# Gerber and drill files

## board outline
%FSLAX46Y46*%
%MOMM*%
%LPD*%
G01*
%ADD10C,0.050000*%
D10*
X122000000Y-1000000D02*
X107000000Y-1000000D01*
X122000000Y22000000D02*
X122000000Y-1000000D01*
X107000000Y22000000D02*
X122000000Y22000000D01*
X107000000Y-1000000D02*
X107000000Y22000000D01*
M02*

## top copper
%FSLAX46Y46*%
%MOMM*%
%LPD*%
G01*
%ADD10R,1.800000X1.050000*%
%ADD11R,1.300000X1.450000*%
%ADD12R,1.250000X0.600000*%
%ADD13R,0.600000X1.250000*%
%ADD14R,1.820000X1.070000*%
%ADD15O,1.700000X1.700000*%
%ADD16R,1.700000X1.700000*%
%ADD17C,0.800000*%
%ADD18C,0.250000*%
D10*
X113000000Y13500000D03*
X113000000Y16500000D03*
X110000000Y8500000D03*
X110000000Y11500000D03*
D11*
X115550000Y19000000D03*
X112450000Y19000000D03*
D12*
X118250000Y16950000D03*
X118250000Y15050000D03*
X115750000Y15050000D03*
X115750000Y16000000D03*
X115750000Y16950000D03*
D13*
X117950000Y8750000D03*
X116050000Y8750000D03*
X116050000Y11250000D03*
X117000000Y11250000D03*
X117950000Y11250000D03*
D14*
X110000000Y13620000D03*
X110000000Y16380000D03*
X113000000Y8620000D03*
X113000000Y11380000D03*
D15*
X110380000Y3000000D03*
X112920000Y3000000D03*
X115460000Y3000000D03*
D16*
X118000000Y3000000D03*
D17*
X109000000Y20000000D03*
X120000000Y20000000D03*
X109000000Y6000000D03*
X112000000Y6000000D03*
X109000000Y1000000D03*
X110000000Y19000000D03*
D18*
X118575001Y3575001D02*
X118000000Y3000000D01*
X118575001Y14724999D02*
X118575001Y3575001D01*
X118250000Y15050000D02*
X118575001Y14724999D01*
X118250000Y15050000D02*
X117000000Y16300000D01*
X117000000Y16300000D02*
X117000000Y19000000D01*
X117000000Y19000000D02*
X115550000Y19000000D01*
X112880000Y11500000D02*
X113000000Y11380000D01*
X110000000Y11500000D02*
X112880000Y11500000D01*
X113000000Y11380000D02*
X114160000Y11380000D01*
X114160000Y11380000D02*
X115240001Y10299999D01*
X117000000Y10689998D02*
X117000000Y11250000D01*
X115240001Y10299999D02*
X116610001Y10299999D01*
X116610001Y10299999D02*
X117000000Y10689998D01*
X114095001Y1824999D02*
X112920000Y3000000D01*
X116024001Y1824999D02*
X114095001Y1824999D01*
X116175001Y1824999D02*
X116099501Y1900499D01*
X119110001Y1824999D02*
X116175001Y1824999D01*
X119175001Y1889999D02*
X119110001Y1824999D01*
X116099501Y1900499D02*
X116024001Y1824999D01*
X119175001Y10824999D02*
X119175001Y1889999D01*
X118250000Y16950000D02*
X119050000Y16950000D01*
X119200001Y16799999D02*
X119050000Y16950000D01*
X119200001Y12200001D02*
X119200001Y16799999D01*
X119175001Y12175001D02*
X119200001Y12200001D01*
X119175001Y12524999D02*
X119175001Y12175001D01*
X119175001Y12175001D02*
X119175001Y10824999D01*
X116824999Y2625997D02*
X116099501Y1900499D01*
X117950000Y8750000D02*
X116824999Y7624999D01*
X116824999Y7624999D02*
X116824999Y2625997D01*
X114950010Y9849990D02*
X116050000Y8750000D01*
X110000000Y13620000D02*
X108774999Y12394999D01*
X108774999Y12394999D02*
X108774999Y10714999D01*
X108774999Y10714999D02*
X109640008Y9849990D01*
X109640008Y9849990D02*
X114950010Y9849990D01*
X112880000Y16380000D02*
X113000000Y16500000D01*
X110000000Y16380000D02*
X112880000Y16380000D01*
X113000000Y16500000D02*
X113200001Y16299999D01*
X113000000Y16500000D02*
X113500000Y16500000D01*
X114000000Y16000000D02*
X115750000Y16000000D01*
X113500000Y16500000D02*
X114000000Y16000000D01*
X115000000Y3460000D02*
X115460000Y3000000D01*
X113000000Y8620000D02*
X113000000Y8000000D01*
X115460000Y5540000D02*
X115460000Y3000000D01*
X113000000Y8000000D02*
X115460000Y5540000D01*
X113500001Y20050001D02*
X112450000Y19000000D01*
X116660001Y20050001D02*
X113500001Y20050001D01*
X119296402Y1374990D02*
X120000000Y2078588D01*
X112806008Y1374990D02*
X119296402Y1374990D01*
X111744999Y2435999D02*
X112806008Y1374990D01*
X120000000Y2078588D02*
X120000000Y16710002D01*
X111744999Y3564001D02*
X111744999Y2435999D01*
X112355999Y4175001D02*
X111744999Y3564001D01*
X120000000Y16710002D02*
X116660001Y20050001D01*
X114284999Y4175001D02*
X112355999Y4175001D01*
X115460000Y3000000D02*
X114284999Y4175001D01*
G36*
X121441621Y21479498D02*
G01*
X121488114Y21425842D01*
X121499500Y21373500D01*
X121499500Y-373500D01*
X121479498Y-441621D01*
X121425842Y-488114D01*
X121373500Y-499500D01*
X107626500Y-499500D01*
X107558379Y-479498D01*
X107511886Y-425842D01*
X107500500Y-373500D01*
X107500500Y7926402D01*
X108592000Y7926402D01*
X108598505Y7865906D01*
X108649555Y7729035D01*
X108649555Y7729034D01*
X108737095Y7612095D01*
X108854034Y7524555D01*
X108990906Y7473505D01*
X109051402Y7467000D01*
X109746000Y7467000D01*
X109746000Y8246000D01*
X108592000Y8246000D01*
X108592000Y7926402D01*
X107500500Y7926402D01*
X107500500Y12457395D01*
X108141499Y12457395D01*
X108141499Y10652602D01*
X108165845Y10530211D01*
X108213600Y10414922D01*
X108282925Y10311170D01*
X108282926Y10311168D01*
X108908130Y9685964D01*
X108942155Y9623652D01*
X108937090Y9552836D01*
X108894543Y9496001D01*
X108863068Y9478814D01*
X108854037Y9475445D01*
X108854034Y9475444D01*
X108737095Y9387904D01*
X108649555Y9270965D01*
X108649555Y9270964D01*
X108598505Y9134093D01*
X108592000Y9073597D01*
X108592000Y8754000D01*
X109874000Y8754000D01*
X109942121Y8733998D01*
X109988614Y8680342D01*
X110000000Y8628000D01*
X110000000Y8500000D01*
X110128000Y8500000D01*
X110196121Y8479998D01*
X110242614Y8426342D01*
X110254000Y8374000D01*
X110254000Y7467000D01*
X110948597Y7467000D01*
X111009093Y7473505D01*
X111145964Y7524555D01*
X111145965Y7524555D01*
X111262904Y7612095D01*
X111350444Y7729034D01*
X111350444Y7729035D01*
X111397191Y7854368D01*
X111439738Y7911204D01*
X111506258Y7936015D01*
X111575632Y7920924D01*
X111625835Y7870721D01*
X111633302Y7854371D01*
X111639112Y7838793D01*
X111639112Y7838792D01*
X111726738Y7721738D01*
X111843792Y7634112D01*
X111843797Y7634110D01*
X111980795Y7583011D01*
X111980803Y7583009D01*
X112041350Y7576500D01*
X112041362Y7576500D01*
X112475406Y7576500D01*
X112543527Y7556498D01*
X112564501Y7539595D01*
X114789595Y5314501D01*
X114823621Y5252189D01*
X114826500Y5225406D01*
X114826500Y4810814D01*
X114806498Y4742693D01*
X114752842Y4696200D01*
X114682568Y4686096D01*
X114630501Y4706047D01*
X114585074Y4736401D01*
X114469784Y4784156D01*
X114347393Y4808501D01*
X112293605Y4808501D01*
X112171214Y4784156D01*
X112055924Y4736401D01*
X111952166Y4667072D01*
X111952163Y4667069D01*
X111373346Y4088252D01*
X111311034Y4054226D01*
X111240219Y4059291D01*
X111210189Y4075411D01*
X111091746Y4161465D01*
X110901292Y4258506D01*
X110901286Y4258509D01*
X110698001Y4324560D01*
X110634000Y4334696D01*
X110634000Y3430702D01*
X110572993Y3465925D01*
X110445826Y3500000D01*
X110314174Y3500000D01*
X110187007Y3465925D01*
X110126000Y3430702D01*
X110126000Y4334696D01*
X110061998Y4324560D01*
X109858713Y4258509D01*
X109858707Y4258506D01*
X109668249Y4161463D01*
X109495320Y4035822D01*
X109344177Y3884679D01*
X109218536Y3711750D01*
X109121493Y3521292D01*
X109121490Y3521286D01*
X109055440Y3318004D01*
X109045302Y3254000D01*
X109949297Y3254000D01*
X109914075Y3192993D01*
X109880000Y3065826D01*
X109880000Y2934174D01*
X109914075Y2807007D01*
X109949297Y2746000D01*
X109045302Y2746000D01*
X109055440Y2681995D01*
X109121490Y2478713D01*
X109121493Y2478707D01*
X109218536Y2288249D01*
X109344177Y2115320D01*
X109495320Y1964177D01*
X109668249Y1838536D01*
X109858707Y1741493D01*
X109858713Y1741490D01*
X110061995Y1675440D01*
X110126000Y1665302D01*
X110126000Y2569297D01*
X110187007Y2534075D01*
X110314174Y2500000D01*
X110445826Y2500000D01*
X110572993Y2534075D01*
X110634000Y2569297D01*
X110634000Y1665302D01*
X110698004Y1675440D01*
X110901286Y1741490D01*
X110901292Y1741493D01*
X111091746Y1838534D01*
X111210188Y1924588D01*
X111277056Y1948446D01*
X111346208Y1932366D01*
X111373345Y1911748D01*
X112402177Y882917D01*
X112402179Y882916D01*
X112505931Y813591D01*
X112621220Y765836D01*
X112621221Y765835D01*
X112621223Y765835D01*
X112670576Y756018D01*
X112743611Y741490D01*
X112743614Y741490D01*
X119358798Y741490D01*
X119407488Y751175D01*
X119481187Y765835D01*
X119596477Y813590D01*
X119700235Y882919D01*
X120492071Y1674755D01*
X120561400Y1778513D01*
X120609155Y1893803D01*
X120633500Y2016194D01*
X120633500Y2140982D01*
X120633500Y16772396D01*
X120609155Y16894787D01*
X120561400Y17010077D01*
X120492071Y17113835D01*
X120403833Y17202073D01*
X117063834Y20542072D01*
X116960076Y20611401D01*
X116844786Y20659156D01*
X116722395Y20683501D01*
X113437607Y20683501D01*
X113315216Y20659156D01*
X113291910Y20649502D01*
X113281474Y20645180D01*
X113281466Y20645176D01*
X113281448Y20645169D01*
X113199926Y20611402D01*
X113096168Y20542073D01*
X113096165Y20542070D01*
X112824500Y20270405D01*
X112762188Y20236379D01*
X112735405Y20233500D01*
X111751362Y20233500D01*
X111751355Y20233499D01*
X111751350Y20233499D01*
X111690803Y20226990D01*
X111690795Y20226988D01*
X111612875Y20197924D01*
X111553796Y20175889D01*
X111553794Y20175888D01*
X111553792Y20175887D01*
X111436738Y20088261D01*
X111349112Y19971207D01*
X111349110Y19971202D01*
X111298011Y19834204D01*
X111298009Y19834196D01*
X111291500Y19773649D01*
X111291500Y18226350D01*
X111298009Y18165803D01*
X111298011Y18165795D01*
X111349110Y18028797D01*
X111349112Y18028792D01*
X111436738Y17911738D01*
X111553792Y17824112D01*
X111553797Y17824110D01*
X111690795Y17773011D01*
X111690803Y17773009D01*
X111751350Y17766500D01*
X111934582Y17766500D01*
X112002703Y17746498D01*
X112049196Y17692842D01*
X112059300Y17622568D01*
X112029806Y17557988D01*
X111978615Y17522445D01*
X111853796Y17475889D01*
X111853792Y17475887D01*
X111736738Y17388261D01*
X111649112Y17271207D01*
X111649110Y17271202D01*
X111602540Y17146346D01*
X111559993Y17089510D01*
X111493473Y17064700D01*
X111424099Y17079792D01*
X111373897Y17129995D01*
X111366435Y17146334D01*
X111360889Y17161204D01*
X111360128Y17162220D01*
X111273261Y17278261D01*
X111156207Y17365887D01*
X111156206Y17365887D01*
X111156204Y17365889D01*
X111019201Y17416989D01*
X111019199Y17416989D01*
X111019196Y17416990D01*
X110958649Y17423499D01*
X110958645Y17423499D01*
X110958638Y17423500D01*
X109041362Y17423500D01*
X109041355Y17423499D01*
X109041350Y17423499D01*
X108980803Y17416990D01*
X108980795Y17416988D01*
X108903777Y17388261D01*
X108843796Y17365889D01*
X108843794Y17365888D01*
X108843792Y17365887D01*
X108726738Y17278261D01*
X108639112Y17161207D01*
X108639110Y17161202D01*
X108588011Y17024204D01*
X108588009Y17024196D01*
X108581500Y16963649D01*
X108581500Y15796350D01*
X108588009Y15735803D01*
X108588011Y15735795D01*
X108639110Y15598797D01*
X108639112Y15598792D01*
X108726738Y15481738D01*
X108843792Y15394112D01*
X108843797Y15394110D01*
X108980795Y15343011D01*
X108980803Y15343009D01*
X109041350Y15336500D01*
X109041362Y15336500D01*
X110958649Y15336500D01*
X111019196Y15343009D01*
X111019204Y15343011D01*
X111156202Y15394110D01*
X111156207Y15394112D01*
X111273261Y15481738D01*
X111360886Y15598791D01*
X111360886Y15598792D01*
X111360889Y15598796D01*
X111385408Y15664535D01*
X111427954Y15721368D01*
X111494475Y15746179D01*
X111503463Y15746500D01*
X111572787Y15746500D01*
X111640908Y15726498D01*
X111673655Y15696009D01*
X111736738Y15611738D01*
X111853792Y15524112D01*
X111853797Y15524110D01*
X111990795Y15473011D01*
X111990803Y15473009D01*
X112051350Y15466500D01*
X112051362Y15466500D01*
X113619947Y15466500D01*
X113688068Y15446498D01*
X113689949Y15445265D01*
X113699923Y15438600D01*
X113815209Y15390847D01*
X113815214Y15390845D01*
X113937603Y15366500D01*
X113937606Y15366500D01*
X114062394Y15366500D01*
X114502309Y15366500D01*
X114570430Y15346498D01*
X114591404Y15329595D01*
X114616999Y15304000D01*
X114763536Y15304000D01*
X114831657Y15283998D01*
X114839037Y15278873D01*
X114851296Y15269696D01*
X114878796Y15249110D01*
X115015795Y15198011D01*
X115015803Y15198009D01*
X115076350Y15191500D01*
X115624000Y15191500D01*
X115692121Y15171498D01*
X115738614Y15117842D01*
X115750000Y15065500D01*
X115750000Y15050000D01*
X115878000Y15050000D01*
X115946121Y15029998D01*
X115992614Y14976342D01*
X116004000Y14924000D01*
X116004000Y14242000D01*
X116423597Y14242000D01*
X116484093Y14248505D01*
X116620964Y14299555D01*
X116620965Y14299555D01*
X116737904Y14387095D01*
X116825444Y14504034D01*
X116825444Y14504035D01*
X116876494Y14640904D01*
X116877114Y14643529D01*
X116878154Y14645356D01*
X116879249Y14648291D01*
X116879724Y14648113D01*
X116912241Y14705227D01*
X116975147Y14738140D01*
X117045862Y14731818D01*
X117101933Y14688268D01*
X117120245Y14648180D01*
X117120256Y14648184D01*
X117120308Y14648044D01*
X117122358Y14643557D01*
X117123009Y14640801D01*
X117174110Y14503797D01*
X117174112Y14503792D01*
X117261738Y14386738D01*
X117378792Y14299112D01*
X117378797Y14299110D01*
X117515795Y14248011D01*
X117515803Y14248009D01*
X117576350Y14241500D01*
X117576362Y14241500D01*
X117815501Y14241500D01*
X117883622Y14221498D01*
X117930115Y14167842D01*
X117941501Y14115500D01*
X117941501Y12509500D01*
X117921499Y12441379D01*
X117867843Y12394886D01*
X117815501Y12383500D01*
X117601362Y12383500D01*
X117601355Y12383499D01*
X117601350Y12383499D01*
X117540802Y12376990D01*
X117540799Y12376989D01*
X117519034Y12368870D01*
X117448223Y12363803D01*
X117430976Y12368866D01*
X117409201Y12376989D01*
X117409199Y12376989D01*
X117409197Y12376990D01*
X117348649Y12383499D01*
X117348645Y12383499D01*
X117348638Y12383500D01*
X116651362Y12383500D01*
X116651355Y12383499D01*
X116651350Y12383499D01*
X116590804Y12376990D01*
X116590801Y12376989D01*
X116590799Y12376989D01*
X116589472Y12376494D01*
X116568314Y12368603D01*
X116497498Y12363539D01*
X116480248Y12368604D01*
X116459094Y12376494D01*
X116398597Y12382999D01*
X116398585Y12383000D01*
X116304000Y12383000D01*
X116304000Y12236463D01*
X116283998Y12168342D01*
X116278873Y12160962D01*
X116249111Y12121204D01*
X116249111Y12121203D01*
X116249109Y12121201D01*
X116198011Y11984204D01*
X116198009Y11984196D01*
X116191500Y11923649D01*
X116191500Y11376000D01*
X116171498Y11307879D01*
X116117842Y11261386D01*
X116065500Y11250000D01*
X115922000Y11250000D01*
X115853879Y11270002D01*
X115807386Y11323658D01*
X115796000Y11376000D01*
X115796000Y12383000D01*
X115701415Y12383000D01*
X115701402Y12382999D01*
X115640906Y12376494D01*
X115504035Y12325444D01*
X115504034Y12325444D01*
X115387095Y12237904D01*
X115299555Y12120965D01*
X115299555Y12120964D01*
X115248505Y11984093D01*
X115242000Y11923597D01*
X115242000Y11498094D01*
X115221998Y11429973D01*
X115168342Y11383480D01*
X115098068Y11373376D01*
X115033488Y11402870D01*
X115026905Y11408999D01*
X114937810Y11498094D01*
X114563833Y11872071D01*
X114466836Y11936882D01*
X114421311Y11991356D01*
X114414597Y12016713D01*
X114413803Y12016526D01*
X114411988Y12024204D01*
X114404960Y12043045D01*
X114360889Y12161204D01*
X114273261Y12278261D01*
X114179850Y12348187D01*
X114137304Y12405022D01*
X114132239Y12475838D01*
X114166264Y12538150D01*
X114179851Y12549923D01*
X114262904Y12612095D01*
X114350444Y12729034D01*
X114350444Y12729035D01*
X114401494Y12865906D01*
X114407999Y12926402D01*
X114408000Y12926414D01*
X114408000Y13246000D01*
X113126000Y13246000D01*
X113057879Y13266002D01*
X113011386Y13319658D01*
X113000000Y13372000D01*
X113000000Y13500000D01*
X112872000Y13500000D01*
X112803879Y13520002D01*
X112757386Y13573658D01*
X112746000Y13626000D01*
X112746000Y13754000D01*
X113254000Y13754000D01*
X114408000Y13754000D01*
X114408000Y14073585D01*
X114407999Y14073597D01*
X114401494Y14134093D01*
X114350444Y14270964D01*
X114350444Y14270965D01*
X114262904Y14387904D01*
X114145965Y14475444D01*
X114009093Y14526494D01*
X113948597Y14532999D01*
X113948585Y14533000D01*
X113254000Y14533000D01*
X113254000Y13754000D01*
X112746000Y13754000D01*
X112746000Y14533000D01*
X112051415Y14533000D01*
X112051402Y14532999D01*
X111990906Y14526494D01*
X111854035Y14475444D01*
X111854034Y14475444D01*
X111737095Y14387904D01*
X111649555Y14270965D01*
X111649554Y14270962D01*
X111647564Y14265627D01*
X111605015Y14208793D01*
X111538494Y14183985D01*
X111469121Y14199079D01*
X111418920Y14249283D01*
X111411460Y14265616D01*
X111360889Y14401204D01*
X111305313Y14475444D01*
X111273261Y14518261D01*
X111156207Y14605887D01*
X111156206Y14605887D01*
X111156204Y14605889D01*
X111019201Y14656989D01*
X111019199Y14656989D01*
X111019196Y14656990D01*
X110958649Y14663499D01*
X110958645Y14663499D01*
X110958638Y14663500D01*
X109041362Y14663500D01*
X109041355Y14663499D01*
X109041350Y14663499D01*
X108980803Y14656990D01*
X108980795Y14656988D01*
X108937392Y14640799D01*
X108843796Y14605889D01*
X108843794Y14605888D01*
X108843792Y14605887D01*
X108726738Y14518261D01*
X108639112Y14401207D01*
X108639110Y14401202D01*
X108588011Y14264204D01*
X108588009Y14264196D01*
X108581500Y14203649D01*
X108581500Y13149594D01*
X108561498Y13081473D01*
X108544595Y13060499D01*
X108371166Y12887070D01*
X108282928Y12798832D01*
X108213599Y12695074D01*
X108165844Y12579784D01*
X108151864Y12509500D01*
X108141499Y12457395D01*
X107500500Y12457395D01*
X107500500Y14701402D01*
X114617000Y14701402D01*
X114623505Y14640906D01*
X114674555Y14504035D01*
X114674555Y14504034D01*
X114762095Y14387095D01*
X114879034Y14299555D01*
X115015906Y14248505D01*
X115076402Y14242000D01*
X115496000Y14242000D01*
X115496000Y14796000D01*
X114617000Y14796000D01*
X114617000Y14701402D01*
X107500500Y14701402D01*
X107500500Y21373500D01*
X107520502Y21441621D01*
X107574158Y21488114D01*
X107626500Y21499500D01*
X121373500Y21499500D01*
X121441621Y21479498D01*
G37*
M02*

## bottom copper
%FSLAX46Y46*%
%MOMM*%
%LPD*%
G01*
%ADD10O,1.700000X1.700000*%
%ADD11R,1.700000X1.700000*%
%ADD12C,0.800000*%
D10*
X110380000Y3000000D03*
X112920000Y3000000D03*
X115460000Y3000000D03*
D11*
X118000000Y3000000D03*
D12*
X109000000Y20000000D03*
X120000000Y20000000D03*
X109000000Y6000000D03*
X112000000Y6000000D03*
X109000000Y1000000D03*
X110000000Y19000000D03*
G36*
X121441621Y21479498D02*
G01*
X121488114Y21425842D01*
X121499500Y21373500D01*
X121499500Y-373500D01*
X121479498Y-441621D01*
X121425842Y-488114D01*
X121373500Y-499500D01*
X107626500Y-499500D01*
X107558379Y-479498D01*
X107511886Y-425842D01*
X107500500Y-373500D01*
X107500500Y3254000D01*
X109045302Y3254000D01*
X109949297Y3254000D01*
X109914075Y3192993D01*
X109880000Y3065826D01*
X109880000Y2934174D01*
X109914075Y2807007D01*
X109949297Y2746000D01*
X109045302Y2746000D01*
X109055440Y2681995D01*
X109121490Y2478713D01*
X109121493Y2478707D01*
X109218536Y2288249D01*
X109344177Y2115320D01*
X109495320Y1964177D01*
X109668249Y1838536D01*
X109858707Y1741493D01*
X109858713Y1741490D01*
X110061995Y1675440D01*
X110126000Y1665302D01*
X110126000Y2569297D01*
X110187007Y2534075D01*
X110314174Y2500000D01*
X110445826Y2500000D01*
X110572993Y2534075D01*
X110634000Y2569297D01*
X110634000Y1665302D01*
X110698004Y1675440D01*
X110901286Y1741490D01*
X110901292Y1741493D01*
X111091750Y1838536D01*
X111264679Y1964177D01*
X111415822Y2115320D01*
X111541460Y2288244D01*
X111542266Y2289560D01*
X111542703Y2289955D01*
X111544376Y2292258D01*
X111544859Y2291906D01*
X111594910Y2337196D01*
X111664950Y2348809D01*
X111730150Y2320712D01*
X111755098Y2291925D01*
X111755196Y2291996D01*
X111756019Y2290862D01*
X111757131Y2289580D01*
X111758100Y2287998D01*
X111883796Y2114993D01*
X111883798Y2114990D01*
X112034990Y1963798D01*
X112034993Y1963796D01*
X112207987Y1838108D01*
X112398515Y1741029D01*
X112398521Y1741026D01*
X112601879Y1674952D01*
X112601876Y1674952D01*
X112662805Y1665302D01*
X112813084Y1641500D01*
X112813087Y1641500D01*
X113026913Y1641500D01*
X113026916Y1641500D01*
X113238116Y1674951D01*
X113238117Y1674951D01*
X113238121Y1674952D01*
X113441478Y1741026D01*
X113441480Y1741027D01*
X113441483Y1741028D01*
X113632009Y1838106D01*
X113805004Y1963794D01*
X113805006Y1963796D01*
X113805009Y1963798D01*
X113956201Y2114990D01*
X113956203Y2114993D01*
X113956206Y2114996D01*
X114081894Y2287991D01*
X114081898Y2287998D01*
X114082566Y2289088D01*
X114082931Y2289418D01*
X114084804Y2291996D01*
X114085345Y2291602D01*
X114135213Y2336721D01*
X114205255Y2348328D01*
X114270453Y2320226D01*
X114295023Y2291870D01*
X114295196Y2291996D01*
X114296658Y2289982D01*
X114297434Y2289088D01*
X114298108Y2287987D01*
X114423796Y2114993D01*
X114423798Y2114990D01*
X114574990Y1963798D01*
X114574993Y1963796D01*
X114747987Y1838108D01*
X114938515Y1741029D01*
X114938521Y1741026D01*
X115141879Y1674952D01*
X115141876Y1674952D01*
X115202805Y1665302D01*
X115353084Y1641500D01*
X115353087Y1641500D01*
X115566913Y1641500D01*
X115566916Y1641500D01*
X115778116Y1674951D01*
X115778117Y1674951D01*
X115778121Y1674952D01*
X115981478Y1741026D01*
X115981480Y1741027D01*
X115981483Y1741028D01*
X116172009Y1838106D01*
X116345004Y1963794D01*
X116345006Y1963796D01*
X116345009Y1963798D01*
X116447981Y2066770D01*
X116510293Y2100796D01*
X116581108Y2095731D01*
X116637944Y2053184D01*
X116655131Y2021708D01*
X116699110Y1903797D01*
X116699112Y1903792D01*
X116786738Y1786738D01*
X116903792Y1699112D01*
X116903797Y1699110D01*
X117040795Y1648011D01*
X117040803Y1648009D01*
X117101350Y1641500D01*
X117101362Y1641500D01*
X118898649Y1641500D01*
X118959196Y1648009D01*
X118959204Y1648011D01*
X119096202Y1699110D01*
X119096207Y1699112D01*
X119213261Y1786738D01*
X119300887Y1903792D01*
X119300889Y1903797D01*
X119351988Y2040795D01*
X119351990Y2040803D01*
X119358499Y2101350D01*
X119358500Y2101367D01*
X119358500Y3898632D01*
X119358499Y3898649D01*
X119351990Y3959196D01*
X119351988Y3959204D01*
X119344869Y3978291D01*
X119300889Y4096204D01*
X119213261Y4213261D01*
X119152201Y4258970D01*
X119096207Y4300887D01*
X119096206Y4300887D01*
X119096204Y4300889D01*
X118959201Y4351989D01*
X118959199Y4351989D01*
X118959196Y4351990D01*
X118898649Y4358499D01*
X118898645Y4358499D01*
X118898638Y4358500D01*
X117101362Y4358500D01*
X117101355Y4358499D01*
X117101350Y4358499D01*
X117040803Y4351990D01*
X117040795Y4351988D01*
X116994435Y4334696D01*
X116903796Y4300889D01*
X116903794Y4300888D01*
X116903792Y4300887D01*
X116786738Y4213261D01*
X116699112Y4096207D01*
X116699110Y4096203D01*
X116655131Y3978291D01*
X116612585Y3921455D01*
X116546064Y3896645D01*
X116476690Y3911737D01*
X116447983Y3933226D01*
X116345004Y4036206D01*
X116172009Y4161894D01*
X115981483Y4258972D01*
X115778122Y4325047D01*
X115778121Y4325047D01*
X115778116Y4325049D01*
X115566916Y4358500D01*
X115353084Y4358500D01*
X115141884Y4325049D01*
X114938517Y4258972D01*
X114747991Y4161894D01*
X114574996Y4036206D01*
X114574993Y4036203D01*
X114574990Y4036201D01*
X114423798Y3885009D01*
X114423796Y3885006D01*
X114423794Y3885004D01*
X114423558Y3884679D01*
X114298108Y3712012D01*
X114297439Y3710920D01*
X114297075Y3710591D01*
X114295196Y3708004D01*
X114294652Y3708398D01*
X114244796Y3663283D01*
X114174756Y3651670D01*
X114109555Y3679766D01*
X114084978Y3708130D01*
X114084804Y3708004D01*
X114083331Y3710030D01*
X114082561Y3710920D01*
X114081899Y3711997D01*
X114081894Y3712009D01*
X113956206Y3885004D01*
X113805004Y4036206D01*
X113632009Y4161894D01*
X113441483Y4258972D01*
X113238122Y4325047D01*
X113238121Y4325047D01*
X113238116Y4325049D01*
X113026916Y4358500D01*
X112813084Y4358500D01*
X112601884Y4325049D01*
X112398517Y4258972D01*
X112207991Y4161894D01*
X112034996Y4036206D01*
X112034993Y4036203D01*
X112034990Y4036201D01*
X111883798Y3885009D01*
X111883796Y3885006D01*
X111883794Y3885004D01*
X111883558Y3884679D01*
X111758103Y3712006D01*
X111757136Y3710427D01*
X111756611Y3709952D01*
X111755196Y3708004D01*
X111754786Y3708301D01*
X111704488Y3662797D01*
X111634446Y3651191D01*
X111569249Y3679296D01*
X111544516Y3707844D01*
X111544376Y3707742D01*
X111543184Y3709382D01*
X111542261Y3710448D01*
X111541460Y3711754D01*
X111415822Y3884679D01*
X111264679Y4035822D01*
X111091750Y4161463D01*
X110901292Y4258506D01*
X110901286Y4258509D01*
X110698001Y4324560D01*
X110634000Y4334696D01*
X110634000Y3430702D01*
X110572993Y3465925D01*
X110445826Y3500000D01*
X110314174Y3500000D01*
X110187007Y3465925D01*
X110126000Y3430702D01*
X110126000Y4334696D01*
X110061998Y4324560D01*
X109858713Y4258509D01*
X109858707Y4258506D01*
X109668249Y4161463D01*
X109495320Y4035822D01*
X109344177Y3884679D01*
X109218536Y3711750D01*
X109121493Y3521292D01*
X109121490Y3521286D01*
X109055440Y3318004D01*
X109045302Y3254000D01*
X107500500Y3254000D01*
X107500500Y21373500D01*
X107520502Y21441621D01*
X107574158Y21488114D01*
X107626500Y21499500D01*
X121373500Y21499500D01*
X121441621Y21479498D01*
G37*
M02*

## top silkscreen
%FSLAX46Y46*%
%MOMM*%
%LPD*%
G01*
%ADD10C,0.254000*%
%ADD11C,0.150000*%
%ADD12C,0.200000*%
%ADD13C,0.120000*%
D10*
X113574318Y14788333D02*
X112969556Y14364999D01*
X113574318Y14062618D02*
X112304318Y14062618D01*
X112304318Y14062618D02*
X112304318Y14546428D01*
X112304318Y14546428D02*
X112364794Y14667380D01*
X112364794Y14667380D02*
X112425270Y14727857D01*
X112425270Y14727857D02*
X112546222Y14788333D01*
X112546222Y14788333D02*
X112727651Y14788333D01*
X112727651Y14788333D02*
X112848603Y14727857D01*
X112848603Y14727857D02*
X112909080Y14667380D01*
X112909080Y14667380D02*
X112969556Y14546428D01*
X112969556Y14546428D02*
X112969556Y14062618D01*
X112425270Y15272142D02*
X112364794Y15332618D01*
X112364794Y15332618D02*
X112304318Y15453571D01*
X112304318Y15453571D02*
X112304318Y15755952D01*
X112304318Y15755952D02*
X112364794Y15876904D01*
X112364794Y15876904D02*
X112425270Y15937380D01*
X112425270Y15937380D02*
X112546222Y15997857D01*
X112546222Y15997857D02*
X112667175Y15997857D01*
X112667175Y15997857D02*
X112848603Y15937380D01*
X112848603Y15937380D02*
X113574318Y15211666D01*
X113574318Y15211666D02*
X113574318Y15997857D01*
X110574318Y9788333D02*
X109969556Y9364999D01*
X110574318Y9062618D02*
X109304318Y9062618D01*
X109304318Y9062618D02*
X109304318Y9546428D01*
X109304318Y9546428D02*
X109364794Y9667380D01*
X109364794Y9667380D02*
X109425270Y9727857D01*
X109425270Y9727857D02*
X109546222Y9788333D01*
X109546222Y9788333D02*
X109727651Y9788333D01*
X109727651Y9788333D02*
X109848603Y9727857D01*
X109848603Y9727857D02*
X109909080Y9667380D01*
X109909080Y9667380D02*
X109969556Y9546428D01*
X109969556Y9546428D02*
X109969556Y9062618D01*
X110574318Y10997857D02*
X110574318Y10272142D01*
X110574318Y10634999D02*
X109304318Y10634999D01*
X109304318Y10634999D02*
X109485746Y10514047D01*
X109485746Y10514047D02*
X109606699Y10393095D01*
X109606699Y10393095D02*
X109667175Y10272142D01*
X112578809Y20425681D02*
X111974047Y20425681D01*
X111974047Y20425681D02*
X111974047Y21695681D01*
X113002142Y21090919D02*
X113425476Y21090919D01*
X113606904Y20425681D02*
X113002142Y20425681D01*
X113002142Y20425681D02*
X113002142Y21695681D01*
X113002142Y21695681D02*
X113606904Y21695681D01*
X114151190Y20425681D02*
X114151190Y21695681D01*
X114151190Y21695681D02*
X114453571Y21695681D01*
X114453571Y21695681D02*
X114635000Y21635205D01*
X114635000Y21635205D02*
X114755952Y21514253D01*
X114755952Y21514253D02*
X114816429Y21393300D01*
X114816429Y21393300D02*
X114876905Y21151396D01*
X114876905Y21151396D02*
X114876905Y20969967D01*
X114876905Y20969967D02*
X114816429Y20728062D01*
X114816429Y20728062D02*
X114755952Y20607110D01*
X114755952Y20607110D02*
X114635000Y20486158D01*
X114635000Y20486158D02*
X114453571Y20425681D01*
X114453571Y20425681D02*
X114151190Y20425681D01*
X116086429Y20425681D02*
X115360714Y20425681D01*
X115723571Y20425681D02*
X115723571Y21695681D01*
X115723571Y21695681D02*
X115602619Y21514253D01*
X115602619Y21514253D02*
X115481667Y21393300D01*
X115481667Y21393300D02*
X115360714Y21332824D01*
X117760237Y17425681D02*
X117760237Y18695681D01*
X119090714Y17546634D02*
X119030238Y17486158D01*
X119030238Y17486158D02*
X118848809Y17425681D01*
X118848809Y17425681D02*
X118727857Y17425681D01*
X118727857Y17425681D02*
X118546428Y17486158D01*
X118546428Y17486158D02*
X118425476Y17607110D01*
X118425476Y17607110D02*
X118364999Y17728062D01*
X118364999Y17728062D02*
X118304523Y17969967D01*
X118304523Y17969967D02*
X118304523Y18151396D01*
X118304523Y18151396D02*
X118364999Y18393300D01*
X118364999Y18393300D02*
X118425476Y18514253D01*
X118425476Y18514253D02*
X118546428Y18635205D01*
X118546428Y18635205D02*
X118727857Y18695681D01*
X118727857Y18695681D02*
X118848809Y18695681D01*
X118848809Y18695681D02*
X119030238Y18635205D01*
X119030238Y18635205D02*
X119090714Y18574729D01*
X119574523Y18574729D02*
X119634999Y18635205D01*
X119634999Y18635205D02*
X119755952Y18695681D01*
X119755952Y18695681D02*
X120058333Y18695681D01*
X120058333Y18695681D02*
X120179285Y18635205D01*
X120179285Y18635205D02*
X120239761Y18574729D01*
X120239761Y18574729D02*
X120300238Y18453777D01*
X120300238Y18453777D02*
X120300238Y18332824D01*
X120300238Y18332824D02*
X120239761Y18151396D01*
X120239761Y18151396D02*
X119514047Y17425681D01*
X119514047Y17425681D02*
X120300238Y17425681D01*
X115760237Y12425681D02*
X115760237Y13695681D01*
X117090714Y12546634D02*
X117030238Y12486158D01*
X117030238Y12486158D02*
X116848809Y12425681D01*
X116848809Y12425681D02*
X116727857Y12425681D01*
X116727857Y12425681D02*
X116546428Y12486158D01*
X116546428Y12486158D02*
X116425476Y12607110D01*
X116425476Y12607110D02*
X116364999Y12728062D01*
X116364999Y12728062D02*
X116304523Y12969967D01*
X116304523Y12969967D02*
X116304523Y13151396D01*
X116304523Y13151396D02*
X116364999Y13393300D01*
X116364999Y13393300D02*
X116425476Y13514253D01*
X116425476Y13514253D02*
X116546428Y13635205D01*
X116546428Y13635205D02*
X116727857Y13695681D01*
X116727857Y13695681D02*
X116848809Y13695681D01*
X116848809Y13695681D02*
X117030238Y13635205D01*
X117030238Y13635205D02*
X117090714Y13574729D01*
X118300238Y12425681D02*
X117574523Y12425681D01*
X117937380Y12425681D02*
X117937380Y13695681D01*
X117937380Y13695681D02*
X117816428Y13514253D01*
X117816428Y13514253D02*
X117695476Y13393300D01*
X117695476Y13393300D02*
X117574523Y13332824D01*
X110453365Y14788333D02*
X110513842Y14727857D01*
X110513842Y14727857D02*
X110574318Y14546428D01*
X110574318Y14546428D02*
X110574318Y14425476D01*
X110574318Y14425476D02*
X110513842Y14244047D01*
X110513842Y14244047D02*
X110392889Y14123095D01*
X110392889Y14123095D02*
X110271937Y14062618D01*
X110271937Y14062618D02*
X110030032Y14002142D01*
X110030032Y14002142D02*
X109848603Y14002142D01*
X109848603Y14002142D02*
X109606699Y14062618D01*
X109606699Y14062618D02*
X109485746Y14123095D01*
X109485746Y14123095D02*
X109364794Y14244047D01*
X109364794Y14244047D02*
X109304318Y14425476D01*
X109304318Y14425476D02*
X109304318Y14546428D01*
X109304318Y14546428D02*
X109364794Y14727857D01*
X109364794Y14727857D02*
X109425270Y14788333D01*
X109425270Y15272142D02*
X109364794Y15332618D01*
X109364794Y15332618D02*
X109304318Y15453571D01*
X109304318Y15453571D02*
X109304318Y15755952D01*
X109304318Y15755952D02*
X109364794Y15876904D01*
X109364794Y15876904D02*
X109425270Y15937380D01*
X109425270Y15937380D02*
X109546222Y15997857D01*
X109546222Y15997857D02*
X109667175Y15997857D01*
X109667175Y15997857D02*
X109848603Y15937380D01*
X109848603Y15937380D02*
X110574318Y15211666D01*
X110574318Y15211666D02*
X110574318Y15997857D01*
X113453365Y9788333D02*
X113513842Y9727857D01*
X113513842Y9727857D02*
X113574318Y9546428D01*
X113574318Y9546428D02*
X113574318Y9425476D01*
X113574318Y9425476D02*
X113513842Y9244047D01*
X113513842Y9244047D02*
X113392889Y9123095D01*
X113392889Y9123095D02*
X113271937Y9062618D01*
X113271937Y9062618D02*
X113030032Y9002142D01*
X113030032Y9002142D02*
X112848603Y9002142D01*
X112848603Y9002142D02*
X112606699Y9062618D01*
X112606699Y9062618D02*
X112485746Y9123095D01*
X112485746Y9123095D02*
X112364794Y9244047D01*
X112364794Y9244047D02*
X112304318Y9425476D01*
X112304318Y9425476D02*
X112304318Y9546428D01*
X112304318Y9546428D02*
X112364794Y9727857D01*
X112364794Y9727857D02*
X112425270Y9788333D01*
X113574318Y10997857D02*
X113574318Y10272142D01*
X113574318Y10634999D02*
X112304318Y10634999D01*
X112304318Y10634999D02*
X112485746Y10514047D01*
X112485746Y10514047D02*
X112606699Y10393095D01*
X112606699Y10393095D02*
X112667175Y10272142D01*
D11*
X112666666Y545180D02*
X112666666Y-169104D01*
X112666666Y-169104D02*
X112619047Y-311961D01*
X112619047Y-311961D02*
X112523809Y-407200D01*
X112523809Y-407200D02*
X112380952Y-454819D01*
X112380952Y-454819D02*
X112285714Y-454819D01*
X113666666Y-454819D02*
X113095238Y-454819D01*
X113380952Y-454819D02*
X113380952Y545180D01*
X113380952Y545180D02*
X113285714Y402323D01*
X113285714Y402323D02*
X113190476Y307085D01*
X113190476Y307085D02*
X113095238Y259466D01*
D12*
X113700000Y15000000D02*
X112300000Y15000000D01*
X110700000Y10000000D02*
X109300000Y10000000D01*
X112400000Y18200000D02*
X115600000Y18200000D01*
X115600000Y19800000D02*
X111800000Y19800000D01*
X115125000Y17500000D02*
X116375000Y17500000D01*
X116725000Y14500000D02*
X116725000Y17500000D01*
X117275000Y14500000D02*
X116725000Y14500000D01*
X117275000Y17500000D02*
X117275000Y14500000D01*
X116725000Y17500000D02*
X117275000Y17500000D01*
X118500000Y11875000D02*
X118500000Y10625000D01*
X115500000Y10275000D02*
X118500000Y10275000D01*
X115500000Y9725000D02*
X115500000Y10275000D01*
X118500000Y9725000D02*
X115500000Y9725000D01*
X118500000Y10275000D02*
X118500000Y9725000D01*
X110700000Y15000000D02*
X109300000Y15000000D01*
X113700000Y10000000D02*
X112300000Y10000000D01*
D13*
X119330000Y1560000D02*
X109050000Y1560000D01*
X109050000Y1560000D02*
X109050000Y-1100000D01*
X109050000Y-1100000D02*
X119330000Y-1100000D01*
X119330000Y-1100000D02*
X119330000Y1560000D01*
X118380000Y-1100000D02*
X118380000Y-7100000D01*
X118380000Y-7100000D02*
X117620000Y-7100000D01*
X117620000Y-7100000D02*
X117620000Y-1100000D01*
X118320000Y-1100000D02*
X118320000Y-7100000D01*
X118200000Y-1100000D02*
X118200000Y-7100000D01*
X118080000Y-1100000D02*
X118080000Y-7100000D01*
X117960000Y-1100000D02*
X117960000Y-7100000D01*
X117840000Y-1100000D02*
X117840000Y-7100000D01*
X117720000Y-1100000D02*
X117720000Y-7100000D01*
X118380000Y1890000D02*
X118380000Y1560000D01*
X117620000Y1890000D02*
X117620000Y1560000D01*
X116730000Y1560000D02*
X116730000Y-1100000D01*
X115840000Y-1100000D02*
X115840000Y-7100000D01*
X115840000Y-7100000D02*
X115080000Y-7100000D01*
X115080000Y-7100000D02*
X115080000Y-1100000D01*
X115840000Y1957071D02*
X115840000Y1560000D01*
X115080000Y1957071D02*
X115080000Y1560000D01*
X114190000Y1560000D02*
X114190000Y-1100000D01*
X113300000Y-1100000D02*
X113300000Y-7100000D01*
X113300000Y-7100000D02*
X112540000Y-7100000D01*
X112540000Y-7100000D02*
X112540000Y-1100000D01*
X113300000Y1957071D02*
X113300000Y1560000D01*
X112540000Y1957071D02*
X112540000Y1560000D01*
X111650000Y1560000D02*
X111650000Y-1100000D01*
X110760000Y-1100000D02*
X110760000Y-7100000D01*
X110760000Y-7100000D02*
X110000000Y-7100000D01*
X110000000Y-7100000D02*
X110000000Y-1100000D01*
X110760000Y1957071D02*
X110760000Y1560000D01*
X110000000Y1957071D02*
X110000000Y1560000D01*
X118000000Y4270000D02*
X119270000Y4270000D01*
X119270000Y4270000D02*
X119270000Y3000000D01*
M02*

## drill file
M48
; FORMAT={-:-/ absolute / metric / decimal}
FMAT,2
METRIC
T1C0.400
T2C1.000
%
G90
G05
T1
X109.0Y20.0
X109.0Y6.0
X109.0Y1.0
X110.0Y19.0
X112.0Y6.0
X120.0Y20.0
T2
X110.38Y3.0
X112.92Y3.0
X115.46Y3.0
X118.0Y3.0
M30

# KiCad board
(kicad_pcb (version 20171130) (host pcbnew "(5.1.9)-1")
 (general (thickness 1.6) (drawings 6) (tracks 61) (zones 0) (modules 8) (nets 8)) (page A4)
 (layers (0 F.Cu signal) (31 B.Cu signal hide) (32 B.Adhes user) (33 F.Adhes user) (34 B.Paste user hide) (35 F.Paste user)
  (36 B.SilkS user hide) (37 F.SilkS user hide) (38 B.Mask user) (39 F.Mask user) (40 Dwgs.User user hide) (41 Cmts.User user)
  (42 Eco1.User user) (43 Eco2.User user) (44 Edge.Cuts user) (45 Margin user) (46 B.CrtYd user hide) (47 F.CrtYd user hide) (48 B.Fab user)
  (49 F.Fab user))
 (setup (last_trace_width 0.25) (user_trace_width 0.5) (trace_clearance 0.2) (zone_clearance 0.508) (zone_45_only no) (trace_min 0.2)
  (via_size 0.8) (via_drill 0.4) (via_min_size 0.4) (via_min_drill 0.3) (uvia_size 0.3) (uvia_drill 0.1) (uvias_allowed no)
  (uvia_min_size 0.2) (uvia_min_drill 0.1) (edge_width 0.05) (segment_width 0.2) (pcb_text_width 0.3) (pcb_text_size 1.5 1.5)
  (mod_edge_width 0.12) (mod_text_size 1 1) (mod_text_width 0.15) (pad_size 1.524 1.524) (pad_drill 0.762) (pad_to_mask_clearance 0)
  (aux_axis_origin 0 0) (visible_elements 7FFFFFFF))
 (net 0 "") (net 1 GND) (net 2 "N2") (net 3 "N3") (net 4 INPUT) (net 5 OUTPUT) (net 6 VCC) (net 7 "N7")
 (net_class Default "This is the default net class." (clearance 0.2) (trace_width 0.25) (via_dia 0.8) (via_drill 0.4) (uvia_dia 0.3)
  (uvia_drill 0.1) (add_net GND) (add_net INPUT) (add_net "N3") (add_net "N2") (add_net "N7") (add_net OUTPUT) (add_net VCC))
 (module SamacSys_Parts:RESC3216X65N (layer F.Cu) (at 113 -15 270)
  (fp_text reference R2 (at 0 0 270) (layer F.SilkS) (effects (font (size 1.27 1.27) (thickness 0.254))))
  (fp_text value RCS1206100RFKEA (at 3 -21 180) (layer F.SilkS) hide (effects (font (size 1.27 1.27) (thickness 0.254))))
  (fp_line (start 0 -0.7) (end 0 0.7) (layer F.SilkS) (width 0.2))
  (pad 2 smd rect (at 1.5 0 270) (size 1.05 1.8) (layers F.Cu F.Paste F.Mask) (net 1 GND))
  (pad 1 smd rect (at -1.5 0 270) (size 1.05 1.8) (layers F.Cu F.Paste F.Mask) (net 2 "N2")))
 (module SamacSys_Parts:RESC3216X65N (layer F.Cu) (at 110 -10 270)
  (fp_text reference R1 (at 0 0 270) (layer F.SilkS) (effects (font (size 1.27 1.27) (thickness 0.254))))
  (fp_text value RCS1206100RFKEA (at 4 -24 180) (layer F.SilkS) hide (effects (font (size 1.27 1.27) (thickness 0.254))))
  (fp_line (start 0 -0.7) (end 0 0.7) (layer F.SilkS) (width 0.2))
  (pad 2 smd rect (at 1.5 0 270) (size 1.05 1.8) (layers F.Cu F.Paste F.Mask) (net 1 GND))
  (pad 1 smd rect (at -1.5 0 270) (size 1.05 1.8) (layers F.Cu F.Paste F.Mask) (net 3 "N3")))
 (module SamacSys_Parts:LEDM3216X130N (layer F.Cu) (at 114 -19)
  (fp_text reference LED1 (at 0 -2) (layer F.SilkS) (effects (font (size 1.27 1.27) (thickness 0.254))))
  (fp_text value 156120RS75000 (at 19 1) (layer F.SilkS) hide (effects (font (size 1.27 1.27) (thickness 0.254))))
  (fp_line (start -1.6 0.8) (end 1.6 0.8) (layer F.SilkS) (width 0.2))
  (fp_line (start 1.6 -0.8) (end -2.2 -0.8) (layer F.SilkS) (width 0.2))
  (pad 2 smd rect (at 1.55 0) (size 1.3 1.45) (layers F.Cu F.Paste F.Mask) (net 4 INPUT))
  (pad 1 smd rect (at -1.55 0) (size 1.3 1.45) (layers F.Cu F.Paste F.Mask) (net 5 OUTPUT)))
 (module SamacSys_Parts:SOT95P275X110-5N (layer F.Cu) (at 117 -16)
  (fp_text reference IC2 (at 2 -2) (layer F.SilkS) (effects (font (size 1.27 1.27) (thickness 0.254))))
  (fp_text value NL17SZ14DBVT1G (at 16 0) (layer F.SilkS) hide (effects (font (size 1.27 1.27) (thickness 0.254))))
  (fp_line (start -1.875 -1.5) (end -0.625 -1.5) (layer F.SilkS) (width 0.2))
  (fp_line (start -0.275 1.5) (end -0.275 -1.5) (layer F.SilkS) (width 0.2))
  (fp_line (start 0.275 1.5) (end -0.275 1.5) (layer F.SilkS) (width 0.2))
  (fp_line (start 0.275 -1.5) (end 0.275 1.5) (layer F.SilkS) (width 0.2))
  (fp_line (start -0.275 -1.5) (end 0.275 -1.5) (layer F.SilkS) (width 0.2))
  (pad 5 smd rect (at 1.25 -0.95 90) (size 0.6 1.25) (layers F.Cu F.Paste F.Mask) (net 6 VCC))
  (pad 4 smd rect (at 1.25 0.95 90) (size 0.6 1.25) (layers F.Cu F.Paste F.Mask) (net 4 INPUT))
  (pad 3 smd rect (at -1.25 0.95 90) (size 0.6 1.25) (layers F.Cu F.Paste F.Mask) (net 1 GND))
  (pad 2 smd rect (at -1.25 0 90) (size 0.6 1.25) (layers F.Cu F.Paste F.Mask) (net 2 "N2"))
  (pad 1 smd rect (at -1.25 -0.95 90) (size 0.6 1.25) (layers F.Cu F.Paste F.Mask)))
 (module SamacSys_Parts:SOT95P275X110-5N (layer F.Cu) (at 117 -10 270)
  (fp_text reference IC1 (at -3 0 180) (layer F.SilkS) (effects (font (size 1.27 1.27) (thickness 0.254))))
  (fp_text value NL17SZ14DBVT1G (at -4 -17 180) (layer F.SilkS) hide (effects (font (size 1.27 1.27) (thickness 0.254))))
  (fp_line (start -1.875 -1.5) (end -0.625 -1.5) (layer F.SilkS) (width 0.2))
  (fp_line (start -0.275 1.5) (end -0.275 -1.5) (layer F.SilkS) (width 0.2))
  (fp_line (start 0.275 1.5) (end -0.275 1.5) (layer F.SilkS) (width 0.2))
  (fp_line (start 0.275 -1.5) (end 0.275 1.5) (layer F.SilkS) (width 0.2))
  (fp_line (start -0.275 -1.5) (end 0.275 -1.5) (layer F.SilkS) (width 0.2))
  (pad 5 smd rect (at 1.25 -0.95) (size 0.6 1.25) (layers F.Cu F.Paste F.Mask) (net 6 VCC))
  (pad 4 smd rect (at 1.25 0.95) (size 0.6 1.25) (layers F.Cu F.Paste F.Mask) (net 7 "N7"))
  (pad 3 smd rect (at -1.25 0.95) (size 0.6 1.25) (layers F.Cu F.Paste F.Mask) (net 1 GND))
  (pad 2 smd rect (at -1.25 0) (size 0.6 1.25) (layers F.Cu F.Paste F.Mask) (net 3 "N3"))
  (pad 1 smd rect (at -1.25 -0.95) (size 0.6 1.25) (layers F.Cu F.Paste F.Mask)))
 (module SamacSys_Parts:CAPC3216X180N (layer F.Cu) (at 110 -15 270)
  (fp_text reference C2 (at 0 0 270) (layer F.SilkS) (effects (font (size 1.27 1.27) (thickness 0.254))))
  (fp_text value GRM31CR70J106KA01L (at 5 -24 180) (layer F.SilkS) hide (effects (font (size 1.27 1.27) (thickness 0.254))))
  (fp_line (start 0 -0.7) (end 0 0.7) (layer F.SilkS) (width 0.2))
  (pad 2 smd rect (at 1.38 0 270) (size 1.07 1.82) (layers F.Cu F.Paste F.Mask) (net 7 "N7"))
  (pad 1 smd rect (at -1.38 0 270) (size 1.07 1.82) (layers F.Cu F.Paste F.Mask) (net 2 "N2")))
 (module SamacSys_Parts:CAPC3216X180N (layer F.Cu) (at 113 -10 270)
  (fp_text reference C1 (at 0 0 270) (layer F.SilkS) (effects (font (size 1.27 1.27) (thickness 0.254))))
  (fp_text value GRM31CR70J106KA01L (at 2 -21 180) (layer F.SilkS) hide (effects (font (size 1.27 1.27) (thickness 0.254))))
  (fp_line (start 0 -0.7) (end 0 0.7) (layer F.SilkS) (width 0.2))
  (pad 2 smd rect (at 1.38 0 270) (size 1.07 1.82) (layers F.Cu F.Paste F.Mask) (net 5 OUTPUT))
  (pad 1 smd rect (at -1.38 0 270) (size 1.07 1.82) (layers F.Cu F.Paste F.Mask) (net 3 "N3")))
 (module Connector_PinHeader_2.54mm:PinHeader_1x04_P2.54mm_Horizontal (layer F.Cu) (at 118 -3 270)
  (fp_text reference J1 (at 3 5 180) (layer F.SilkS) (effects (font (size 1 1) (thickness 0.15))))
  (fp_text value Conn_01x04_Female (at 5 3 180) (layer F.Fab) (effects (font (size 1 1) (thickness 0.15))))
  (fp_line (start 1.44 -1.33) (end 1.44 8.95) (layer F.SilkS) (width 0.12))
  (fp_line (start 1.44 8.95) (end 4.1 8.95) (layer F.SilkS) (width 0.12))
  (fp_line (start 4.1 8.95) (end 4.1 -1.33) (layer F.SilkS) (width 0.12))
  (fp_line (start 4.1 -1.33) (end 1.44 -1.33) (layer F.SilkS) (width 0.12))
  (fp_line (start 4.1 -0.38) (end 10.1 -0.38) (layer F.SilkS) (width 0.12))
  (fp_line (start 10.1 -0.38) (end 10.1 0.38) (layer F.SilkS) (width 0.12))
  (fp_line (start 10.1 0.38) (end 4.1 0.38) (layer F.SilkS) (width 0.12))
  (fp_line (start 4.1 -0.32) (end 10.1 -0.32) (layer F.SilkS) (width 0.12))
  (fp_line (start 4.1 -0.2) (end 10.1 -0.2) (layer F.SilkS) (width 0.12))
  (fp_line (start 4.1 -0.08) (end 10.1 -0.08) (layer F.SilkS) (width 0.12))
  (fp_line (start 4.1 0.04) (end 10.1 0.04) (layer F.SilkS) (width 0.12))
  (fp_line (start 4.1 0.16) (end 10.1 0.16) (layer F.SilkS) (width 0.12))
  (fp_line (start 4.1 0.28) (end 10.1 0.28) (layer F.SilkS) (width 0.12))
  (fp_line (start 1.11 -0.38) (end 1.44 -0.38) (layer F.SilkS) (width 0.12))
  (fp_line (start 1.11 0.38) (end 1.44 0.38) (layer F.SilkS) (width 0.12))
  (fp_line (start 1.44 1.27) (end 4.1 1.27) (layer F.SilkS) (width 0.12))
  (fp_line (start 4.1 2.16) (end 10.1 2.16) (layer F.SilkS) (width 0.12))
  (fp_line (start 10.1 2.16) (end 10.1 2.92) (layer F.SilkS) (width 0.12))
  (fp_line (start 10.1 2.92) (end 4.1 2.92) (layer F.SilkS) (width 0.12))
  (fp_line (start 1.042929 2.16) (end 1.44 2.16) (layer F.SilkS) (width 0.12))
  (fp_line (start 1.042929 2.92) (end 1.44 2.92) (layer F.SilkS) (width 0.12))
  (fp_line (start 1.44 3.81) (end 4.1 3.81) (layer F.SilkS) (width 0.12))
  (fp_line (start 4.1 4.7) (end 10.1 4.7) (layer F.SilkS) (width 0.12))
  (fp_line (start 10.1 4.7) (end 10.1 5.46) (layer F.SilkS) (width 0.12))
  (fp_line (start 10.1 5.46) (end 4.1 5.46) (layer F.SilkS) (width 0.12))
  (fp_line (start 1.042929 4.7) (end 1.44 4.7) (layer F.SilkS) (width 0.12))
  (fp_line (start 1.042929 5.46) (end 1.44 5.46) (layer F.SilkS) (width 0.12))
  (fp_line (start 1.44 6.35) (end 4.1 6.35) (layer F.SilkS) (width 0.12))
  (fp_line (start 4.1 7.24) (end 10.1 7.24) (layer F.SilkS) (width 0.12))
  (fp_line (start 10.1 7.24) (end 10.1 8) (layer F.SilkS) (width 0.12))
  (fp_line (start 10.1 8) (end 4.1 8) (layer F.SilkS) (width 0.12))
  (fp_line (start 1.042929 7.24) (end 1.44 7.24) (layer F.SilkS) (width 0.12))
  (fp_line (start 1.042929 8) (end 1.44 8) (layer F.SilkS) (width 0.12))
  (fp_line (start -1.27 0) (end -1.27 -1.27) (layer F.SilkS) (width 0.12))
  (fp_line (start -1.27 -1.27) (end 0 -1.27) (layer F.SilkS) (width 0.12))
  (pad 4 thru_hole oval (at 0 7.62 270) (size 1.7 1.7) (drill 1) (layers *.Cu *.Mask) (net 1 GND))
  (pad 3 thru_hole oval (at 0 5.08 270) (size 1.7 1.7) (drill 1) (layers *.Cu *.Mask) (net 6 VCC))
  (pad 2 thru_hole oval (at 0 2.54 270) (size 1.7 1.7) (drill 1) (layers *.Cu *.Mask) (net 5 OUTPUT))
  (pad 1 thru_hole rect (at 0 0 270) (size 1.7 1.7) (drill 1) (layers *.Cu *.Mask) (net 4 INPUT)))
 (gr_line (start 122 1) (end 107 1) (layer Edge.Cuts) (width 0.05))
 (gr_line (start 122 -22) (end 122 1) (layer Edge.Cuts) (width 0.05))
 (gr_line (start 107 -22) (end 122 -22) (layer Edge.Cuts) (width 0.05))
 (gr_line (start 107 1) (end 107 -22) (layer Edge.Cuts) (width 0.05))
 (segment (start 118.575001 -3.575001) (end 118 -3) (width 0.25) (layer F.Cu) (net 4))
 (segment (start 118.575001 -14.724999) (end 118.575001 -3.575001) (width 0.25) (layer F.Cu) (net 4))
 (segment (start 118.25 -15.05) (end 118.575001 -14.724999) (width 0.25) (layer F.Cu) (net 4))
 (segment (start 118.25 -15.05) (end 117 -16.3) (width 0.25) (layer F.Cu) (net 4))
 (segment (start 117 -16.3) (end 117 -19) (width 0.25) (layer F.Cu) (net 4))
 (segment (start 117 -19) (end 115.55 -19) (width 0.25) (layer F.Cu) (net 4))
 (segment (start 112.88 -11.5) (end 113 -11.38) (width 0.25) (layer F.Cu) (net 3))
 (segment (start 110 -11.5) (end 112.88 -11.5) (width 0.25) (layer F.Cu) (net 3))
 (segment (start 113 -11.38) (end 114.16 -11.38) (width 0.25) (layer F.Cu) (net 3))
 (segment (start 114.16 -11.38) (end 115.240001 -10.299999) (width 0.25) (layer F.Cu) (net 3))
 (segment (start 117 -10.689998) (end 117 -11.25) (width 0.25) (layer F.Cu) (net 3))
 (segment (start 115.240001 -10.299999) (end 116.610001 -10.299999) (width 0.25) (layer F.Cu) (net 3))
 (segment (start 116.610001 -10.299999) (end 117 -10.689998) (width 0.25) (layer F.Cu) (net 3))
 (via (at 109 -20) (size 0.8) (drill 0.4) (layers F.Cu B.Cu) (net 1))
 (via (at 120 -20) (size 0.8) (drill 0.4) (layers F.Cu B.Cu) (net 1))
 (via (at 109 -6) (size 0.8) (drill 0.4) (layers F.Cu B.Cu) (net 1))
 (via (at 112 -6) (size 0.8) (drill 0.4) (layers F.Cu B.Cu) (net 1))
 (via (at 109 -1) (size 0.8) (drill 0.4) (layers F.Cu B.Cu) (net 1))
 (via (at 110 -19) (size 0.8) (drill 0.4) (layers F.Cu B.Cu) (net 1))
 (segment (start 114.095001 -1.824999) (end 112.92 -3) (width 0.25) (layer F.Cu) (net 6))
 (segment (start 116.024001 -1.824999) (end 114.095001 -1.824999) (width 0.25) (layer F.Cu) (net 6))
 (segment (start 116.175001 -1.824999) (end 116.099501 -1.900499) (width 0.25) (layer F.Cu) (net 6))
 (segment (start 119.110001 -1.824999) (end 116.175001 -1.824999) (width 0.25) (layer F.Cu) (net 6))
 (segment (start 119.175001 -1.889999) (end 119.110001 -1.824999) (width 0.25) (layer F.Cu) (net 6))
 (segment (start 116.099501 -1.900499) (end 116.024001 -1.824999) (width 0.25) (layer F.Cu) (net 6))
 (segment (start 119.175001 -10.824999) (end 119.175001 -1.889999) (width 0.25) (layer F.Cu) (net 6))
 (segment (start 118.25 -16.95) (end 119.05 -16.95) (width 0.25) (layer F.Cu) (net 6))
 (segment (start 119.200001 -16.799999) (end 119.05 -16.95) (width 0.25) (layer F.Cu) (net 6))
 (segment (start 119.200001 -12.200001) (end 119.200001 -16.799999) (width 0.25) (layer F.Cu) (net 6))
 (segment (start 119.175001 -12.175001) (end 119.200001 -12.200001) (width 0.25) (layer F.Cu) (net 6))
 (segment (start 119.175001 -12.524999) (end 119.175001 -12.175001) (width 0.25) (layer F.Cu) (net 6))
 (segment (start 119.175001 -12.175001) (end 119.175001 -10.824999) (width 0.25) (layer F.Cu) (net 6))
 (segment (start 116.824999 -2.625997) (end 116.099501 -1.900499) (width 0.25) (layer F.Cu) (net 6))
 (segment (start 117.95 -8.75) (end 116.824999 -7.624999) (width 0.25) (layer F.Cu) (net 6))
 (segment (start 116.824999 -7.624999) (end 116.824999 -2.625997) (width 0.25) (layer F.Cu) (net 6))
 (segment (start 114.95001 -9.84999) (end 116.05 -8.75) (width 0.25) (layer F.Cu) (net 7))
 (segment (start 110 -13.62) (end 108.774999 -12.394999) (width 0.25) (layer F.Cu) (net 7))
 (segment (start 108.774999 -12.394999) (end 108.774999 -10.714999) (width 0.25) (layer F.Cu) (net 7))
 (segment (start 108.774999 -10.714999) (end 109.640008 -9.84999) (width 0.25) (layer F.Cu) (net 7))
 (segment (start 109.640008 -9.84999) (end 114.95001 -9.84999) (width 0.25) (layer F.Cu) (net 7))
 (segment (start 112.88 -16.38) (end 113 -16.5) (width 0.25) (layer F.Cu) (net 2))
 (segment (start 110 -16.38) (end 112.88 -16.38) (width 0.25) (layer F.Cu) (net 2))
 (segment (start 113 -16.5) (end 113.200001 -16.299999) (width 0.25) (layer F.Cu) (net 2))
 (segment (start 113 -16.5) (end 113.5 -16.5) (width 0.25) (layer F.Cu) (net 2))
 (segment (start 114 -16) (end 115.75 -16) (width 0.25) (layer F.Cu) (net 2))
 (segment (start 113.5 -16.5) (end 114 -16) (width 0.25) (layer F.Cu) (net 2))
 (segment (start 115 -3.46) (end 115.46 -3) (width 0.25) (layer F.Cu) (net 5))
 (segment (start 113 -8.62) (end 113 -8) (width 0.25) (layer F.Cu) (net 5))
 (segment (start 115.46 -5.54) (end 115.46 -3) (width 0.25) (layer F.Cu) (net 5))
 (segment (start 113 -8) (end 115.46 -5.54) (width 0.25) (layer F.Cu) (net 5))
 (segment (start 113.500001 -20.050001) (end 112.45 -19) (width 0.25) (layer F.Cu) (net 5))
 (segment (start 116.660001 -20.050001) (end 113.500001 -20.050001) (width 0.25) (layer F.Cu) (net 5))
 (segment (start 119.296402 -1.37499) (end 120 -2.078588) (width 0.25) (layer F.Cu) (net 5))
 (segment (start 112.806008 -1.37499) (end 119.296402 -1.37499) (width 0.25) (layer F.Cu) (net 5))
 (segment (start 111.744999 -2.435999) (end 112.806008 -1.37499) (width 0.25) (layer F.Cu) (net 5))
 (segment (start 120 -2.078588) (end 120 -16.710002) (width 0.25) (layer F.Cu) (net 5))
 (segment (start 111.744999 -3.564001) (end 111.744999 -2.435999) (width 0.25) (layer F.Cu) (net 5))
 (segment (start 112.355999 -4.175001) (end 111.744999 -3.564001) (width 0.25) (layer F.Cu) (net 5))
 (segment (start 120 -16.710002) (end 116.660001 -20.050001) (width 0.25) (layer F.Cu) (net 5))
 (segment (start 114.284999 -4.175001) (end 112.355999 -4.175001) (width 0.25) (layer F.Cu) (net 5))
 (segment (start 115.46 -3) (end 114.284999 -4.175001) (width 0.25) (layer F.Cu) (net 5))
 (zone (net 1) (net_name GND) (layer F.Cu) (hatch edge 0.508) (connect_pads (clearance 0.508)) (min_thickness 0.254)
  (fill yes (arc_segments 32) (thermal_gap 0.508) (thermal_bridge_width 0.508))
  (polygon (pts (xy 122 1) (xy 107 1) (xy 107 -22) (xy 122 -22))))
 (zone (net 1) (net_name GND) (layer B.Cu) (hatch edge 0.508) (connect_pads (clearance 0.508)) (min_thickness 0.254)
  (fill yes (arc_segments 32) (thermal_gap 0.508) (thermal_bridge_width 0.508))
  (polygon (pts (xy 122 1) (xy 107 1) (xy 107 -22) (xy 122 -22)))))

